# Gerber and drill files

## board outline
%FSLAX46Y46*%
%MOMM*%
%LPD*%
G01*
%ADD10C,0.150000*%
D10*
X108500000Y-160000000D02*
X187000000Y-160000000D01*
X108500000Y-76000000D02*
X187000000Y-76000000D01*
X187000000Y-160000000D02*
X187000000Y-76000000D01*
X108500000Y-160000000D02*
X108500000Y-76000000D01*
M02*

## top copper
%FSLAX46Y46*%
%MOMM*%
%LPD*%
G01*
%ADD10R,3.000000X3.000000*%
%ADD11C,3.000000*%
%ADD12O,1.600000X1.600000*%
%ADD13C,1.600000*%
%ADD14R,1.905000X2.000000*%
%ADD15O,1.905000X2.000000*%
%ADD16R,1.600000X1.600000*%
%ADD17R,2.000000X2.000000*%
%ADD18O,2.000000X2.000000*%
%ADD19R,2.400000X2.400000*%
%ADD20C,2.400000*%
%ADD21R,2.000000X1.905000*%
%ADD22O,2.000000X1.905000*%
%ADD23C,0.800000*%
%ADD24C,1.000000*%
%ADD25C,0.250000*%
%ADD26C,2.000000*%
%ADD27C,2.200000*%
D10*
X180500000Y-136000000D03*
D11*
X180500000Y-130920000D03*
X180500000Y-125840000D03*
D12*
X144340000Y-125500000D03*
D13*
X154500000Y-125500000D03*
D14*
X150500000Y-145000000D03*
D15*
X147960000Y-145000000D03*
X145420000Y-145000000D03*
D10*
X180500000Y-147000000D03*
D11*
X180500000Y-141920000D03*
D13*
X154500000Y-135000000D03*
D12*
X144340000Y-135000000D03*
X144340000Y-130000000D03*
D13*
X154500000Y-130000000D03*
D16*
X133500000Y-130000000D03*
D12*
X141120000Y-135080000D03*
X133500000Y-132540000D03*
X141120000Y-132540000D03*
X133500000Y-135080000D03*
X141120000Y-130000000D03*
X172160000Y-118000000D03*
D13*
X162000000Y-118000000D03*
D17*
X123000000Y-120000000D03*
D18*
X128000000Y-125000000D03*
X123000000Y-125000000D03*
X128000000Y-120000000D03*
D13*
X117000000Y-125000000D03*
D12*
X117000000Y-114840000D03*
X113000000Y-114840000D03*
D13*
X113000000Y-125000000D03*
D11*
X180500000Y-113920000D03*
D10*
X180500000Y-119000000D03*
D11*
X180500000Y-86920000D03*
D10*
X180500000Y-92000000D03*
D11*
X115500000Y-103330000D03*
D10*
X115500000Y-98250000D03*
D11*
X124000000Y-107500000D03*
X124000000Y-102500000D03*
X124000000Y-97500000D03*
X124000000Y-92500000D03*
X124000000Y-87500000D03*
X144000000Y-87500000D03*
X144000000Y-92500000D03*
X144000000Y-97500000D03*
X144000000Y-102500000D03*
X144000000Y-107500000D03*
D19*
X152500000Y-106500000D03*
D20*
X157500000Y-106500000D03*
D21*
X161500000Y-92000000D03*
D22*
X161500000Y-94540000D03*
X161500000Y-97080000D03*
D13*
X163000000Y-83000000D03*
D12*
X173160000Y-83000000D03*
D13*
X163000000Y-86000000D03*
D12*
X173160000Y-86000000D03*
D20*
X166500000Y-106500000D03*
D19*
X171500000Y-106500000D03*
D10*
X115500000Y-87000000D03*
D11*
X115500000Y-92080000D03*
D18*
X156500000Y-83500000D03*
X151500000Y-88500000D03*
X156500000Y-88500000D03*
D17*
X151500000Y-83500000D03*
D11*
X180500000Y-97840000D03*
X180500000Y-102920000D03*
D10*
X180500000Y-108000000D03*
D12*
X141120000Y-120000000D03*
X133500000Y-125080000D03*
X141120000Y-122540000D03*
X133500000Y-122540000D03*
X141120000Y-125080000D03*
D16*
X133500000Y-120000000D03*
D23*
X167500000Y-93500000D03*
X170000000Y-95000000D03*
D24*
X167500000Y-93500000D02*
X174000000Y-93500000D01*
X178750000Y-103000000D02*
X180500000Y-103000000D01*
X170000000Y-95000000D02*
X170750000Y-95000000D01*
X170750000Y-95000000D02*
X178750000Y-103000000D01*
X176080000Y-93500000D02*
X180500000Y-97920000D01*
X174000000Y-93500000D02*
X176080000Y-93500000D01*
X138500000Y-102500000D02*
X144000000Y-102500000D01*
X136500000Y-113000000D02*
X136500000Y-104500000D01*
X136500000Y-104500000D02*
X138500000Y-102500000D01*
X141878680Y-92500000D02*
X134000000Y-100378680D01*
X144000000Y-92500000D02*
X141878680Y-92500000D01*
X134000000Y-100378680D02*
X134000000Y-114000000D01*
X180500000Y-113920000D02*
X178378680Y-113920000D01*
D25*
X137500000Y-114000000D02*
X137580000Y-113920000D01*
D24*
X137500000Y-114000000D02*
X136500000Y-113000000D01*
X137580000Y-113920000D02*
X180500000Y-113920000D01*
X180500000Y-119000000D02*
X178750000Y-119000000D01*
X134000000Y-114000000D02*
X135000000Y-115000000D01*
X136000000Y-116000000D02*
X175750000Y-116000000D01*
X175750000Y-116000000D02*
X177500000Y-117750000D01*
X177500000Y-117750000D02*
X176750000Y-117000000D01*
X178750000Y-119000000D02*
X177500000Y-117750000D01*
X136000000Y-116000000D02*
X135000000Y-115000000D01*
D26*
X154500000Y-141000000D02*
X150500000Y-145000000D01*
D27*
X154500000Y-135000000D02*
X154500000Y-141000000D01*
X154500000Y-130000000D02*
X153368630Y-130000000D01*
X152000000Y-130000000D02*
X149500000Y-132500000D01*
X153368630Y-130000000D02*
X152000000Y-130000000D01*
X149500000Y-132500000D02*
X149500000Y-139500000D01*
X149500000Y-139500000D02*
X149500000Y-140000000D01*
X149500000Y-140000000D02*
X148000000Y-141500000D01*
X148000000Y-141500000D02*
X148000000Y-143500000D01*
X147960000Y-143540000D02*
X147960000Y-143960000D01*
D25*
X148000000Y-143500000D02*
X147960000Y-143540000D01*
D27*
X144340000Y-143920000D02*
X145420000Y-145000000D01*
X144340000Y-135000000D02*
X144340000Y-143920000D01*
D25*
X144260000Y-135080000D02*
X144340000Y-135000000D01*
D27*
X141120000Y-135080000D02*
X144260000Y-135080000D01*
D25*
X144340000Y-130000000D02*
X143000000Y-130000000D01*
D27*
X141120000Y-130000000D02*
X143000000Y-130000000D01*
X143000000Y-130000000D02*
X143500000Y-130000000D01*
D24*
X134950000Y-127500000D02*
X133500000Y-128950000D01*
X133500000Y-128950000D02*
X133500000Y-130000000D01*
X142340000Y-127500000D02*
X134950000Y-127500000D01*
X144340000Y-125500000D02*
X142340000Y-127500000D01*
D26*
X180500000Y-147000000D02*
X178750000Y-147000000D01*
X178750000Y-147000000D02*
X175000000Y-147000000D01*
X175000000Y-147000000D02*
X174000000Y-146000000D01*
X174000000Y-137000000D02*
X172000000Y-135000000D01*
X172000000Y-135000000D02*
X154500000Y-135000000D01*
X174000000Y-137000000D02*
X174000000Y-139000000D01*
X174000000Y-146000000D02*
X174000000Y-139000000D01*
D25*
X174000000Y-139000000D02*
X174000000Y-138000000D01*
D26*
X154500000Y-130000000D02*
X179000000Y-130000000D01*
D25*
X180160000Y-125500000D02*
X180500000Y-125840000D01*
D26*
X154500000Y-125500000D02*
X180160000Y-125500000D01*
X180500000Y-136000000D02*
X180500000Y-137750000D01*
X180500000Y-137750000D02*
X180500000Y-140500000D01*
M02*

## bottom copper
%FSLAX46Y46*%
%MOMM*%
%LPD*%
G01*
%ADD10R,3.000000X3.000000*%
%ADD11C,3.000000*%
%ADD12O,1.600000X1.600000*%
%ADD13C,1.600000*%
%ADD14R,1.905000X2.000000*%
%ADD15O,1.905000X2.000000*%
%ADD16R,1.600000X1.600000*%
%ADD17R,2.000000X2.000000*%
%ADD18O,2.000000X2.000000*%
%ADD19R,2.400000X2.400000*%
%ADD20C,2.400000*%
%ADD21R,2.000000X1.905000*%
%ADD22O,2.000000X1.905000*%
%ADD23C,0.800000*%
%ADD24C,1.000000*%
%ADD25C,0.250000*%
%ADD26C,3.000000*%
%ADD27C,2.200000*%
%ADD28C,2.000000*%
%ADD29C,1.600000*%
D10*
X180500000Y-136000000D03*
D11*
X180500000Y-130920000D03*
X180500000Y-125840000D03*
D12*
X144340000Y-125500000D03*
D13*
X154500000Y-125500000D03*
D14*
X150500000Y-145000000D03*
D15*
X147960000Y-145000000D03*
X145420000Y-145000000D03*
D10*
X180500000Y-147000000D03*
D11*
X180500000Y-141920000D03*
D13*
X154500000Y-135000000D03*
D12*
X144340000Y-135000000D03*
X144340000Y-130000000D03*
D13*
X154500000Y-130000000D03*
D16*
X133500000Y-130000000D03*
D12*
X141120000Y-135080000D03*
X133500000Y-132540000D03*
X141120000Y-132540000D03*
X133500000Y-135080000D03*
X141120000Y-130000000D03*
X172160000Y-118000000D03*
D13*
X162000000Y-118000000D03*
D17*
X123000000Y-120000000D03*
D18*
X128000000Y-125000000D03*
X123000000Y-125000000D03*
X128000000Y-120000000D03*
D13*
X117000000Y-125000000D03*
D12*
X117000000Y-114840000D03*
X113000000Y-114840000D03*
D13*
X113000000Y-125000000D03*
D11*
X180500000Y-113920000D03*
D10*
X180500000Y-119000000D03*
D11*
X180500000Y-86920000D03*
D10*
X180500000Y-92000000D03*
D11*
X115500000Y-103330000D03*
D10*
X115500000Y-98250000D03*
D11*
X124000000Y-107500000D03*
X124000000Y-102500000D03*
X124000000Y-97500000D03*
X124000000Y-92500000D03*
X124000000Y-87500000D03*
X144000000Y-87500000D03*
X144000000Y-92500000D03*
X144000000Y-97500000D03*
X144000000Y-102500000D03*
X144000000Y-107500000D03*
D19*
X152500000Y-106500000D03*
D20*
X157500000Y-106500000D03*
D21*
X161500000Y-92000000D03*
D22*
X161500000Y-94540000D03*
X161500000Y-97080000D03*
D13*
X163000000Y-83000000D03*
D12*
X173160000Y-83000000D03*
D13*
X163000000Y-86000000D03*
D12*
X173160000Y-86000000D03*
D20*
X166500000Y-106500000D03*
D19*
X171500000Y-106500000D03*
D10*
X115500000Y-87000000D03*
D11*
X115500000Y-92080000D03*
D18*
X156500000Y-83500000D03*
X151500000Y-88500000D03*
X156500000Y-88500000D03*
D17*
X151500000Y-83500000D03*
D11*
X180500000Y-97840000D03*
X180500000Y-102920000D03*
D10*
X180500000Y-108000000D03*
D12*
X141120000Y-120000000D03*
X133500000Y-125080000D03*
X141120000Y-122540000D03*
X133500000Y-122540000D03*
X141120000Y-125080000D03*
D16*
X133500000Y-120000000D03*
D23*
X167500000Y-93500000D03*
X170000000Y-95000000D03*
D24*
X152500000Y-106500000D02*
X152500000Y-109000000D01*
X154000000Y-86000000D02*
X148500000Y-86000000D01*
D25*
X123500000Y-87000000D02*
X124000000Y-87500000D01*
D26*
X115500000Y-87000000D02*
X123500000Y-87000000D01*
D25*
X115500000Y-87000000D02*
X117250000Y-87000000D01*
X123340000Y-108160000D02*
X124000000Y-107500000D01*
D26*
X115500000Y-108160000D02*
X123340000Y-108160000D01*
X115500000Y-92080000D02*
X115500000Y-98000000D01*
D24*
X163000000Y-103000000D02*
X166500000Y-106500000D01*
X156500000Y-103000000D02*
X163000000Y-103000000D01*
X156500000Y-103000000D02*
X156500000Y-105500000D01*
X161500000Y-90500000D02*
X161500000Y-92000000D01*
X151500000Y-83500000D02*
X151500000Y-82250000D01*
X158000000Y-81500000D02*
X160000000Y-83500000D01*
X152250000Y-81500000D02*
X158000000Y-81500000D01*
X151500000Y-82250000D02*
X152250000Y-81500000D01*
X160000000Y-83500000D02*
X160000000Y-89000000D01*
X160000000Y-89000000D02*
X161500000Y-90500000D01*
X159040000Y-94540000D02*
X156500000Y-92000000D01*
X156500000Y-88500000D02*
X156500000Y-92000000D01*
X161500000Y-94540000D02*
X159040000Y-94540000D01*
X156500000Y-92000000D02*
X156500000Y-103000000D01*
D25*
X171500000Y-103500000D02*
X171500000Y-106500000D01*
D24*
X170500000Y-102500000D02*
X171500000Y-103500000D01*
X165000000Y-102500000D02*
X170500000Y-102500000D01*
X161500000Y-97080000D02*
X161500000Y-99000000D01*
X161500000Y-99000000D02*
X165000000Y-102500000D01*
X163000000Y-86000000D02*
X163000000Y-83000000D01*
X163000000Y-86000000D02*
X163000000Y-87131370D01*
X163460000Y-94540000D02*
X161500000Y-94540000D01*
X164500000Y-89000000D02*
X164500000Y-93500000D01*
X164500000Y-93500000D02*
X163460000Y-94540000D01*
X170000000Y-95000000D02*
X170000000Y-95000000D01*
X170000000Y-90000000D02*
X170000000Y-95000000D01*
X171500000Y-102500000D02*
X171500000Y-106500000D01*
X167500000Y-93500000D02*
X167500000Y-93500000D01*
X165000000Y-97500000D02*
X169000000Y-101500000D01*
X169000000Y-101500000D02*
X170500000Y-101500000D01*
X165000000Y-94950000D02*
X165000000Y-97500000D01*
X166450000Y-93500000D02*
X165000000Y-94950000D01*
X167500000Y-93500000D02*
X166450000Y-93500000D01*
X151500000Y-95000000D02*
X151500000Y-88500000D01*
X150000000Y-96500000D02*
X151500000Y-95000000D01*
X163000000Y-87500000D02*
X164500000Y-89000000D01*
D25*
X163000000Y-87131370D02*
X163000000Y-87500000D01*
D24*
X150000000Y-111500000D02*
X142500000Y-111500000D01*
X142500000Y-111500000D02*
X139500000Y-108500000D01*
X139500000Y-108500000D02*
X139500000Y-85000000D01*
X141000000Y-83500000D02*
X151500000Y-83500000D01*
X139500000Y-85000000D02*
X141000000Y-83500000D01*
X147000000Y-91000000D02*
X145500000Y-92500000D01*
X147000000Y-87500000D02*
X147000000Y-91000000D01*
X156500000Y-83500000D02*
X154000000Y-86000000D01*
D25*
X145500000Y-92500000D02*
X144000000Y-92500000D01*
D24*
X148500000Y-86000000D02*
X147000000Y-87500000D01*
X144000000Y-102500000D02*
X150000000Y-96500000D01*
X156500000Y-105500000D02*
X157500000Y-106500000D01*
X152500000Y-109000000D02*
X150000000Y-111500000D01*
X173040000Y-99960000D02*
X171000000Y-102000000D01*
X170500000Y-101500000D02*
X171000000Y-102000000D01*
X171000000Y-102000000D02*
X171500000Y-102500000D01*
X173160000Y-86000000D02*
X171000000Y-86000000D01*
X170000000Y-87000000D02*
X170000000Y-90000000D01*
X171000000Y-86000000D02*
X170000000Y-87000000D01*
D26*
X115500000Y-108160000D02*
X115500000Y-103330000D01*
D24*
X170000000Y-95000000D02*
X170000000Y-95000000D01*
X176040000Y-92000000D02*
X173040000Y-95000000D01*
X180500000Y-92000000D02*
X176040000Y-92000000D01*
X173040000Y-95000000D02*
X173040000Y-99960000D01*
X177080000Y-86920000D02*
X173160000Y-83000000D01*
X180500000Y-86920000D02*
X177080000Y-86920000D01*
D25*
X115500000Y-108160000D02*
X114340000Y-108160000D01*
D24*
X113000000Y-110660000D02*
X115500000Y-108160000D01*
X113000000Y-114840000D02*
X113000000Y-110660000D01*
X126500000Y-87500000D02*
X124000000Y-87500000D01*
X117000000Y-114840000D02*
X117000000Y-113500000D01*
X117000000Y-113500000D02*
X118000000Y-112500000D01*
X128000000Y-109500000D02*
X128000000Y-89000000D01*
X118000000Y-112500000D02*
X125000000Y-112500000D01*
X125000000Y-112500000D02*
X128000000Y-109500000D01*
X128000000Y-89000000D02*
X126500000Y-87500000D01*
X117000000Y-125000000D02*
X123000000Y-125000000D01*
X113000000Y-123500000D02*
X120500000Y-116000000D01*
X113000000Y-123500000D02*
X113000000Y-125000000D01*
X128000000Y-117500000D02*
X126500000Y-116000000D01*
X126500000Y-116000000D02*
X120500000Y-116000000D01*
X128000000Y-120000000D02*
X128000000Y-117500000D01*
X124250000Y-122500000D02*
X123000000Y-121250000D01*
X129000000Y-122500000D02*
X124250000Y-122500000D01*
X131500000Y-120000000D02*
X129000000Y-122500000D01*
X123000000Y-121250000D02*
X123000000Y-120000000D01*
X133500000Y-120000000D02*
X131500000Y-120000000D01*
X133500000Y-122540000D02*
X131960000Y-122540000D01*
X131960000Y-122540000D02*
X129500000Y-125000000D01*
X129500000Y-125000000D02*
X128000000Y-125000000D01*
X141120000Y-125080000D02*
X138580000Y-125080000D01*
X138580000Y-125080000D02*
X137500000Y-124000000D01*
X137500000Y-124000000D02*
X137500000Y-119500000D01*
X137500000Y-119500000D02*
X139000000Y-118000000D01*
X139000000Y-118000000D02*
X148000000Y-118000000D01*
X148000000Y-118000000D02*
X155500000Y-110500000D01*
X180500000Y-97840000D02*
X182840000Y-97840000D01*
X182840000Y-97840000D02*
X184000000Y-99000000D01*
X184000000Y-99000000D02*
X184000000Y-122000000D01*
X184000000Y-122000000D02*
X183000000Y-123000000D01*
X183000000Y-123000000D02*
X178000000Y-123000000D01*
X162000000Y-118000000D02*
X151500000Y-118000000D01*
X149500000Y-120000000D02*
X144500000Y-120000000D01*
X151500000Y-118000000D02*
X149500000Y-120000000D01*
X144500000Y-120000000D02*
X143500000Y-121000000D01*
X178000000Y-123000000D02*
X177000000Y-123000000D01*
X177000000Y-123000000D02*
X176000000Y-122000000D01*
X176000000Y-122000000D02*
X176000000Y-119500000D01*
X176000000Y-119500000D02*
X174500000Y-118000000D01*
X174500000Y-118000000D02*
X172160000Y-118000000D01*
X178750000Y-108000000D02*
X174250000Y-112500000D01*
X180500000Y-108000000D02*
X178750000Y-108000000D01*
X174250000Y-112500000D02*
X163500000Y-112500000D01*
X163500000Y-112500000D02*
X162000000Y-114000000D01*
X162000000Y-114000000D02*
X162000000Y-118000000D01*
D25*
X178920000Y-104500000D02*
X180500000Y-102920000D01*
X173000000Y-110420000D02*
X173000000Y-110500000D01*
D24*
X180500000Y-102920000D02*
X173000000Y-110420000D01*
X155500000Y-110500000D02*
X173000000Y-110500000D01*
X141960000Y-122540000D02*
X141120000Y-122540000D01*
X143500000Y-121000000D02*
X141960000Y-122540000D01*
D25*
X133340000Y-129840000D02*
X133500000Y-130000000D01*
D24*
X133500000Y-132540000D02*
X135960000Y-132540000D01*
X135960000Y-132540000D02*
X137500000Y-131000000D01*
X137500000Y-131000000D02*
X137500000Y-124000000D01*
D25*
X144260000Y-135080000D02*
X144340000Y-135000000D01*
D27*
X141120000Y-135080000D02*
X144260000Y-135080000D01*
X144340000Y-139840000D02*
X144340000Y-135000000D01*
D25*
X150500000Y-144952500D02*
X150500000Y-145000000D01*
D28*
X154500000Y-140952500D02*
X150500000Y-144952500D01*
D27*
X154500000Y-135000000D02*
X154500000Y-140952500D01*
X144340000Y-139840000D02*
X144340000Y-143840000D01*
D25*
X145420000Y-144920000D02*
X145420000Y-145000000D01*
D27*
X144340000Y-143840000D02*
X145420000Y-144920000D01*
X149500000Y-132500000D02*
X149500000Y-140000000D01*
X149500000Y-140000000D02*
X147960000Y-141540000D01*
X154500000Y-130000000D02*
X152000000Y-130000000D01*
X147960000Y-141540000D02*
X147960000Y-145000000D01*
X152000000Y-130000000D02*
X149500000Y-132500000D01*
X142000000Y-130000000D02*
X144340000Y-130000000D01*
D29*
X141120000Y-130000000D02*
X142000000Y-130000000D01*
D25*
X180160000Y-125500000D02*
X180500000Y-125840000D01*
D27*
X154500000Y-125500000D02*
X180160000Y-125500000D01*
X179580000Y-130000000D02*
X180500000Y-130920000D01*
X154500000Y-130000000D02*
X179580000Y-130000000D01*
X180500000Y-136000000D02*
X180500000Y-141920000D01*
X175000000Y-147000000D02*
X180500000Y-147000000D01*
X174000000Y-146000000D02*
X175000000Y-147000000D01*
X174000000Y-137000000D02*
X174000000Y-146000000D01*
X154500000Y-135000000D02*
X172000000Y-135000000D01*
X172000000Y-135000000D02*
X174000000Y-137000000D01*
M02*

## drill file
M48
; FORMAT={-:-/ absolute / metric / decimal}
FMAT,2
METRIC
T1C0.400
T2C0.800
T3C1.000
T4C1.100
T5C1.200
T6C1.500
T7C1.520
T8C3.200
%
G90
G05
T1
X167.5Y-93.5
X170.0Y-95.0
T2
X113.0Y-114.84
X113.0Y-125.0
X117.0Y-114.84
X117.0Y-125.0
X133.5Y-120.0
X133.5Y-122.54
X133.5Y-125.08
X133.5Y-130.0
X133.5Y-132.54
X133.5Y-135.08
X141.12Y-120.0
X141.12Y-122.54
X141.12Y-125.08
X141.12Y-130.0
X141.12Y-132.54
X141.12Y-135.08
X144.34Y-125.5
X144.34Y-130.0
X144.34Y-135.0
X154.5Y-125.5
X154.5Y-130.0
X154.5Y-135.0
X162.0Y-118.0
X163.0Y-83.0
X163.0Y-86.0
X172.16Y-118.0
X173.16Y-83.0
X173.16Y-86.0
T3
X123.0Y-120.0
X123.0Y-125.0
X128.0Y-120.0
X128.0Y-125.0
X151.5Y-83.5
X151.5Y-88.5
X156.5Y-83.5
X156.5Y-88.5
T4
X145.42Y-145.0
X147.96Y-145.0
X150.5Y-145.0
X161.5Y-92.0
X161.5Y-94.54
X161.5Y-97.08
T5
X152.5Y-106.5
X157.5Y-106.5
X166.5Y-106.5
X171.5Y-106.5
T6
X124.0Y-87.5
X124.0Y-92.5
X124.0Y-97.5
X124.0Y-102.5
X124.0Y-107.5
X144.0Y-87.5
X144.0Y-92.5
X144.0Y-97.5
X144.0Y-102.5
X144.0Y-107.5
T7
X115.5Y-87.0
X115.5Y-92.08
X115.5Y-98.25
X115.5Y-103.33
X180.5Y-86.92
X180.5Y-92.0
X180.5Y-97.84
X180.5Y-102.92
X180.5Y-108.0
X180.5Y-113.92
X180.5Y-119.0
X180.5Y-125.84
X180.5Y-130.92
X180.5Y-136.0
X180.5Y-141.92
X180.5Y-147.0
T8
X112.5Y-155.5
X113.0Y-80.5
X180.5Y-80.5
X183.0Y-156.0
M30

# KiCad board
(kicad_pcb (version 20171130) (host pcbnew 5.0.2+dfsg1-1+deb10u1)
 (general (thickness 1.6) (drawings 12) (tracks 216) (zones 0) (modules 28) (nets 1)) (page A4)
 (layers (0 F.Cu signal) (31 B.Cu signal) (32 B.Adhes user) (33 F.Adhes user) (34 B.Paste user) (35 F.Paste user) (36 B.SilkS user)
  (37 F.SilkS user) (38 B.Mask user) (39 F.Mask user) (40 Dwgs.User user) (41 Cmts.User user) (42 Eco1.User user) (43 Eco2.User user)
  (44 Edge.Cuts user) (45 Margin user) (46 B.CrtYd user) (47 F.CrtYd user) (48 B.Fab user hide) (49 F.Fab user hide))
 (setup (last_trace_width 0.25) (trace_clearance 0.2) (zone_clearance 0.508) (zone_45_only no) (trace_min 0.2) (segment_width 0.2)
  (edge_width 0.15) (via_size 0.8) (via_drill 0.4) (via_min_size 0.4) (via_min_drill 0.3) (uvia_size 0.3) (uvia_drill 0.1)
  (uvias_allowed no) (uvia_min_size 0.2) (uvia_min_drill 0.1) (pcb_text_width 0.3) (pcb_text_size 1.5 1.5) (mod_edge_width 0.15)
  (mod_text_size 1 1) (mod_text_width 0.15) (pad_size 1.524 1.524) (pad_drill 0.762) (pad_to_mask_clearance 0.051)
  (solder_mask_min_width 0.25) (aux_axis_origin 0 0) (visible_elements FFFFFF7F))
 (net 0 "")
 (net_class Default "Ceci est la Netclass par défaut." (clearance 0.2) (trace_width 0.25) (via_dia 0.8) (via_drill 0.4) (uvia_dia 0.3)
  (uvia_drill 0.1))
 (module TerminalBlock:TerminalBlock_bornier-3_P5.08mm (layer F.Cu) (at 180.5 136 90)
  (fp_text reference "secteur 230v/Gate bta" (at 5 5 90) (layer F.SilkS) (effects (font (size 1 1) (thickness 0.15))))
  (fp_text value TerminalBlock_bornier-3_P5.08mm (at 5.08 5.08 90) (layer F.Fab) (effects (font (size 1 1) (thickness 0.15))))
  (pad 1 thru_hole rect (at 0 0 90) (size 3 3) (drill 1.52) (layers *.Cu *.Mask))
  (pad 2 thru_hole circle (at 5.08 0 90) (size 3 3) (drill 1.52) (layers *.Cu *.Mask))
  (pad 3 thru_hole circle (at 10.16 0 90) (size 3 3) (drill 1.52) (layers *.Cu *.Mask)))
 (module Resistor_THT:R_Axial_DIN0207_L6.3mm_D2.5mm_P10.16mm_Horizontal (layer F.Cu) (at 154.5 125.5 180)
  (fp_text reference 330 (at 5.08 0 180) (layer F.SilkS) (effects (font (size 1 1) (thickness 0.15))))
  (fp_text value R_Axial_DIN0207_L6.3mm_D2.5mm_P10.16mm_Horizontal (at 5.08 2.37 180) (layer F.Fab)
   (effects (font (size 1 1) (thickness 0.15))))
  (pad 2 thru_hole oval (at 10.16 0 180) (size 1.6 1.6) (drill 0.8) (layers *.Cu *.Mask))
  (pad 1 thru_hole circle (at 0 0 180) (size 1.6 1.6) (drill 0.8) (layers *.Cu *.Mask)))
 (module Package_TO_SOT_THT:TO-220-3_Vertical (layer F.Cu) (at 150.5 145 180)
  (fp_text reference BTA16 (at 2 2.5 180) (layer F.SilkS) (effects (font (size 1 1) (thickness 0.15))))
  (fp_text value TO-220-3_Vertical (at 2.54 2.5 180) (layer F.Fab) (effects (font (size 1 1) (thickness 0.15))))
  (pad 1 thru_hole rect (at 0 0 180) (size 1.905 2) (drill 1.1) (layers *.Cu *.Mask))
  (pad 2 thru_hole oval (at 2.54 0 180) (size 1.905 2) (drill 1.1) (layers *.Cu *.Mask))
  (pad 3 thru_hole oval (at 5.08 0 180) (size 1.905 2) (drill 1.1) (layers *.Cu *.Mask)))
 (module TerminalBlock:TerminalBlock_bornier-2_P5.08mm (layer F.Cu) (at 180.5 147 90)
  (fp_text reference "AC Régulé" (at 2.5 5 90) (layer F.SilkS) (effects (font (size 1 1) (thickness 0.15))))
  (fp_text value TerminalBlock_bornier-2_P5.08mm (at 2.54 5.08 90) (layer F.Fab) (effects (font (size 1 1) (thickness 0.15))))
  (pad 1 thru_hole rect (at 0 0 90) (size 3 3) (drill 1.52) (layers *.Cu *.Mask))
  (pad 2 thru_hole circle (at 5.08 0 90) (size 3 3) (drill 1.52) (layers *.Cu *.Mask)))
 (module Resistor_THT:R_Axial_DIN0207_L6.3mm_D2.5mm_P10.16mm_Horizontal (layer F.Cu) (at 154.5 135 180)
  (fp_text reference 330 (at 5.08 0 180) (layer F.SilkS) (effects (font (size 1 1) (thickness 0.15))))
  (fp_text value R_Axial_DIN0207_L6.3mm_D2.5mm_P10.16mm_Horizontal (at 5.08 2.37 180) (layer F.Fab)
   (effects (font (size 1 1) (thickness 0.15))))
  (pad 1 thru_hole circle (at 0 0 180) (size 1.6 1.6) (drill 0.8) (layers *.Cu *.Mask))
  (pad 2 thru_hole oval (at 10.16 0 180) (size 1.6 1.6) (drill 0.8) (layers *.Cu *.Mask)))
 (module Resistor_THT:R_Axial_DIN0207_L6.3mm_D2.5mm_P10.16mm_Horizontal (layer F.Cu) (at 154.5 130 180)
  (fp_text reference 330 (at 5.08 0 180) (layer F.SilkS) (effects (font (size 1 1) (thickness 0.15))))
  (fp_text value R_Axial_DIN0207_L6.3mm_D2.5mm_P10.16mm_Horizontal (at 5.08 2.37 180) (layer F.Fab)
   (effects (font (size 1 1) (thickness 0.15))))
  (pad 2 thru_hole oval (at 10.16 0 180) (size 1.6 1.6) (drill 0.8) (layers *.Cu *.Mask))
  (pad 1 thru_hole circle (at 0 0 180) (size 1.6 1.6) (drill 0.8) (layers *.Cu *.Mask)))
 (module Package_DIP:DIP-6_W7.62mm (layer F.Cu) (at 133.5 130)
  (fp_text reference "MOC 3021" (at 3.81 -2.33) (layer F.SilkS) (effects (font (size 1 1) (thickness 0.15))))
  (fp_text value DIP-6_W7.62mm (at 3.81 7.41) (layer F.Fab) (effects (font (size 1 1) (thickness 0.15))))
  (pad 1 thru_hole rect (at 0 0) (size 1.6 1.6) (drill 0.8) (layers *.Cu *.Mask))
  (pad 4 thru_hole oval (at 7.62 5.08) (size 1.6 1.6) (drill 0.8) (layers *.Cu *.Mask))
  (pad 2 thru_hole oval (at 0 2.54) (size 1.6 1.6) (drill 0.8) (layers *.Cu *.Mask))
  (pad 5 thru_hole oval (at 7.62 2.54) (size 1.6 1.6) (drill 0.8) (layers *.Cu *.Mask))
  (pad 3 thru_hole oval (at 0 5.08) (size 1.6 1.6) (drill 0.8) (layers *.Cu *.Mask))
  (pad 6 thru_hole oval (at 7.62 0) (size 1.6 1.6) (drill 0.8) (layers *.Cu *.Mask)))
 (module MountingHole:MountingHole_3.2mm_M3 (layer F.Cu) (at 183 156)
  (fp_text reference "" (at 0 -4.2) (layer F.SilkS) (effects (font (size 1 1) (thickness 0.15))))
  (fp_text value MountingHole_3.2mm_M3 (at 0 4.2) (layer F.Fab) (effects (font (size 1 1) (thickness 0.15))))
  (pad 1 np_thru_hole circle (at 0 0) (size 3.2 3.2) (drill 3.2) (layers *.Cu *.Mask)))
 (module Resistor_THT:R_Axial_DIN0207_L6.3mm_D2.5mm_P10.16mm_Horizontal (layer F.Cu) (at 162 118)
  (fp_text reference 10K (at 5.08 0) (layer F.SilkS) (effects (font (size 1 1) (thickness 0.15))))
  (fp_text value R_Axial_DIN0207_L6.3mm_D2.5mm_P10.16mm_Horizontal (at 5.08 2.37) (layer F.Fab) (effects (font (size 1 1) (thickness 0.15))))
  (pad 2 thru_hole oval (at 10.16 0) (size 1.6 1.6) (drill 0.8) (layers *.Cu *.Mask))
  (pad 1 thru_hole circle (at 0 0) (size 1.6 1.6) (drill 0.8) (layers *.Cu *.Mask)))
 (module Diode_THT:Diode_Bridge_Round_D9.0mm (layer F.Cu) (at 123 120)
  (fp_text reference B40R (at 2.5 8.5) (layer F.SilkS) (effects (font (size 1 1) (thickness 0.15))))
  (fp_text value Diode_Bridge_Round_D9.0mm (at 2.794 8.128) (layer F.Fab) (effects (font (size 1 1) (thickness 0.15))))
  (pad 1 thru_hole rect (at 0 0) (size 2 2) (drill 1) (layers *.Cu *.Mask))
  (pad 3 thru_hole oval (at 5 5) (size 2 2) (drill 1) (layers *.Cu *.Mask))
  (pad 2 thru_hole oval (at 0 5) (size 2 2) (drill 1) (layers *.Cu *.Mask))
  (pad 4 thru_hole oval (at 5 0) (size 2 2) (drill 1) (layers *.Cu *.Mask)))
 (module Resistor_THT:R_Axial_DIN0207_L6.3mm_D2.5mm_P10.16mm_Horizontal (layer F.Cu) (at 117 125 90)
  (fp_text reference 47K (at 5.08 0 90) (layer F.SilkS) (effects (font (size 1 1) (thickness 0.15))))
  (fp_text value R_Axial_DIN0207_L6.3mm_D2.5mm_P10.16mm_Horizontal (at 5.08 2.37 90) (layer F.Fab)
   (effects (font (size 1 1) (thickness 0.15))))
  (pad 1 thru_hole circle (at 0 0 90) (size 1.6 1.6) (drill 0.8) (layers *.Cu *.Mask))
  (pad 2 thru_hole oval (at 10.16 0 90) (size 1.6 1.6) (drill 0.8) (layers *.Cu *.Mask)))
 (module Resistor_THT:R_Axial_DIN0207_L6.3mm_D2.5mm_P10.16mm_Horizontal (layer F.Cu) (at 113 125 90)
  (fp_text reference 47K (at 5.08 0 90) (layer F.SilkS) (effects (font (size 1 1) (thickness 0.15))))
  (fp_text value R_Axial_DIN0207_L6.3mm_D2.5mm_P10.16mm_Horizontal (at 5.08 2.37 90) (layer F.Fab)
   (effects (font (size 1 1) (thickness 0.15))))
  (pad 2 thru_hole oval (at 10.16 0 90) (size 1.6 1.6) (drill 0.8) (layers *.Cu *.Mask))
  (pad 1 thru_hole circle (at 0 0 90) (size 1.6 1.6) (drill 0.8) (layers *.Cu *.Mask)))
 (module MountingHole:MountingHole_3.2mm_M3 (layer F.Cu) (at 180.5 80.5)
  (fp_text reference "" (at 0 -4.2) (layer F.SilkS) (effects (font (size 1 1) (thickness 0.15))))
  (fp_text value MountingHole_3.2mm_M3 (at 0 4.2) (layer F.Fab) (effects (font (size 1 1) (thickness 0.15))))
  (pad 1 np_thru_hole circle (at 0 0) (size 3.2 3.2) (drill 3.2) (layers *.Cu *.Mask)))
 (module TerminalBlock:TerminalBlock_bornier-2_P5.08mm (layer F.Cu) (at 180.5 119 90)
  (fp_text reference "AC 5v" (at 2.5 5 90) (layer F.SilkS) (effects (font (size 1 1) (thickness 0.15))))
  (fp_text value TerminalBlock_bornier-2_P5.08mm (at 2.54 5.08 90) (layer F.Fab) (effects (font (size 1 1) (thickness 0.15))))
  (pad 2 thru_hole circle (at 5.08 0 90) (size 3 3) (drill 1.52) (layers *.Cu *.Mask))
  (pad 1 thru_hole rect (at 0 0 90) (size 3 3) (drill 1.52) (layers *.Cu *.Mask)))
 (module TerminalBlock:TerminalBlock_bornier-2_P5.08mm (layer F.Cu) (at 180.5 92 90)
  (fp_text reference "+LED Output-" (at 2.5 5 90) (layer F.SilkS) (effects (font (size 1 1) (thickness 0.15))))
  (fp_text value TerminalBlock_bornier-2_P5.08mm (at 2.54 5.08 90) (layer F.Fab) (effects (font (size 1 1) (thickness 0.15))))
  (pad 2 thru_hole circle (at 5.08 0 90) (size 3 3) (drill 1.52) (layers *.Cu *.Mask))
  (pad 1 thru_hole rect (at 0 0 90) (size 3 3) (drill 1.52) (layers *.Cu *.Mask)))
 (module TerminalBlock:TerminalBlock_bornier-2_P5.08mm (layer F.Cu) (at 115.5 98.25 270)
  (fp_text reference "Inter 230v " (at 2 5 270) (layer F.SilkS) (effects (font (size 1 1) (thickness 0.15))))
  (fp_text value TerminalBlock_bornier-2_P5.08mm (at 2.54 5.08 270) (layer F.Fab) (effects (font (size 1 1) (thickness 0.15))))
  (pad 2 thru_hole circle (at 5.08 0 270) (size 3 3) (drill 1.52) (layers *.Cu *.Mask))
  (pad 1 thru_hole rect (at 0 0 270) (size 3 3) (drill 1.52) (layers *.Cu *.Mask)))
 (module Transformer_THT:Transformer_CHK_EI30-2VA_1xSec (layer F.Cu) (at 124 107.5)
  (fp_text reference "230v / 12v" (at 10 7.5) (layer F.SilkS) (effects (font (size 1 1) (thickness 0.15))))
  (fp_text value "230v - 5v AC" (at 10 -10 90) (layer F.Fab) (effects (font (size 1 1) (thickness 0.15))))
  (pad 1 thru_hole circle (at 0 0) (size 3 3) (drill 1.5) (layers *.Cu *.Mask))
  (pad 2 thru_hole circle (at 0 -5) (size 3 3) (drill 1.5) (layers *.Cu *.Mask))
  (pad 3 thru_hole circle (at 0 -10) (size 3 3) (drill 1.5) (layers *.Cu *.Mask))
  (pad 4 thru_hole circle (at 0 -15) (size 3 3) (drill 1.5) (layers *.Cu *.Mask))
  (pad 5 thru_hole circle (at 0 -20) (size 3 3) (drill 1.5) (layers *.Cu *.Mask))
  (pad 6 thru_hole circle (at 20 -20) (size 3 3) (drill 1.5) (layers *.Cu *.Mask))
  (pad 7 thru_hole circle (at 20 -15) (size 3 3) (drill 1.5) (layers *.Cu *.Mask))
  (pad 8 thru_hole circle (at 20 -10) (size 3 3) (drill 1.5) (layers *.Cu *.Mask))
  (pad 9 thru_hole circle (at 20 -5) (size 3 3) (drill 1.5) (layers *.Cu *.Mask))
  (pad 10 thru_hole circle (at 20 0) (size 3 3) (drill 1.5) (layers *.Cu *.Mask)))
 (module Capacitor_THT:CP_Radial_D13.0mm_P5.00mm (layer F.Cu) (at 152.5 106.5)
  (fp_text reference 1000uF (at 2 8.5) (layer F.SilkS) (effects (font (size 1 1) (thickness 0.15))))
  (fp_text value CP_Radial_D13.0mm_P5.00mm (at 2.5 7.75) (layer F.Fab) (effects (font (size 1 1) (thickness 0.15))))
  (pad 1 thru_hole rect (at 0 0) (size 2.4 2.4) (drill 1.2) (layers *.Cu *.Mask))
  (pad 2 thru_hole circle (at 5 0) (size 2.4 2.4) (drill 1.2) (layers *.Cu *.Mask)))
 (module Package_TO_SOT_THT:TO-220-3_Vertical (layer F.Cu) (at 161.5 92 270)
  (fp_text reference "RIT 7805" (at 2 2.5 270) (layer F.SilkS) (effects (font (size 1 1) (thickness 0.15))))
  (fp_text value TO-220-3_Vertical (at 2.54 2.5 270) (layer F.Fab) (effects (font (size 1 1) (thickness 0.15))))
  (pad 1 thru_hole rect (at 0 0 270) (size 1.905 2) (drill 1.1) (layers *.Cu *.Mask))
  (pad 2 thru_hole oval (at 2.54 0 270) (size 1.905 2) (drill 1.1) (layers *.Cu *.Mask))
  (pad 3 thru_hole oval (at 5.08 0 270) (size 1.905 2) (drill 1.1) (layers *.Cu *.Mask)))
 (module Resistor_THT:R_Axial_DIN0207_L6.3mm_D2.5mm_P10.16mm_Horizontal (layer F.Cu) (at 163 83)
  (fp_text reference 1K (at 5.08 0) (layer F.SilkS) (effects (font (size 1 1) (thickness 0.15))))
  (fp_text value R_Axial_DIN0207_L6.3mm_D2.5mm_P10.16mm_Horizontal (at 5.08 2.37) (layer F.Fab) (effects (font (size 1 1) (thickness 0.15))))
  (pad 1 thru_hole circle (at 0 0) (size 1.6 1.6) (drill 0.8) (layers *.Cu *.Mask))
  (pad 2 thru_hole oval (at 10.16 0) (size 1.6 1.6) (drill 0.8) (layers *.Cu *.Mask)))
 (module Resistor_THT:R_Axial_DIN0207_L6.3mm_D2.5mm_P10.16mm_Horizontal (layer F.Cu) (at 163 86)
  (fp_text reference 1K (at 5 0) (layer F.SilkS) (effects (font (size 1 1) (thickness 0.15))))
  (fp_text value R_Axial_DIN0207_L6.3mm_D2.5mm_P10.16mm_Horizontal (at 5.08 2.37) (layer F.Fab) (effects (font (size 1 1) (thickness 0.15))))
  (pad 1 thru_hole circle (at 0 0) (size 1.6 1.6) (drill 0.8) (layers *.Cu *.Mask))
  (pad 2 thru_hole oval (at 10.16 0) (size 1.6 1.6) (drill 0.8) (layers *.Cu *.Mask)))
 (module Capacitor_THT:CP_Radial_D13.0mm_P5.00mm (layer F.Cu) (at 171.5 106.5 180)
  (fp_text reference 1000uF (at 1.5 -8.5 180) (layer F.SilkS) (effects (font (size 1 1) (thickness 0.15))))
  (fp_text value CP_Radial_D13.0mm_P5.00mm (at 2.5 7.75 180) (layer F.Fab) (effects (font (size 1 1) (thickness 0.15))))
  (pad 2 thru_hole circle (at 5 0 180) (size 2.4 2.4) (drill 1.2) (layers *.Cu *.Mask))
  (pad 1 thru_hole rect (at 0 0 180) (size 2.4 2.4) (drill 1.2) (layers *.Cu *.Mask)))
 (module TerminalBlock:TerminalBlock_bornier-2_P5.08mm (layer F.Cu) (at 115.5 87 270)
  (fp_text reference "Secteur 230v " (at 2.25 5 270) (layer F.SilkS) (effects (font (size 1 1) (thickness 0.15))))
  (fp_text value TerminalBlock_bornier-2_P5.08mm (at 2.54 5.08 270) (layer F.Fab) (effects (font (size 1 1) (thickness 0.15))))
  (pad 1 thru_hole rect (at 0 0 270) (size 3 3) (drill 1.52) (layers *.Cu *.Mask))
  (pad 2 thru_hole circle (at 5.08 0 270) (size 3 3) (drill 1.52) (layers *.Cu *.Mask)))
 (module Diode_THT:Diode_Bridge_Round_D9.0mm (layer F.Cu) (at 151.5 83.5)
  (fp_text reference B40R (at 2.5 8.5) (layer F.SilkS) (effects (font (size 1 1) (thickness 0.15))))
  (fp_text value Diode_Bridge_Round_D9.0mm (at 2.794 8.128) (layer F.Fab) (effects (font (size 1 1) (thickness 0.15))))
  (pad 4 thru_hole oval (at 5 0) (size 2 2) (drill 1) (layers *.Cu *.Mask))
  (pad 2 thru_hole oval (at 0 5) (size 2 2) (drill 1) (layers *.Cu *.Mask))
  (pad 3 thru_hole oval (at 5 5) (size 2 2) (drill 1) (layers *.Cu *.Mask))
  (pad 1 thru_hole rect (at 0 0) (size 2 2) (drill 1) (layers *.Cu *.Mask)))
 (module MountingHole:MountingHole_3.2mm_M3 (layer F.Cu) (at 112.5 155.5)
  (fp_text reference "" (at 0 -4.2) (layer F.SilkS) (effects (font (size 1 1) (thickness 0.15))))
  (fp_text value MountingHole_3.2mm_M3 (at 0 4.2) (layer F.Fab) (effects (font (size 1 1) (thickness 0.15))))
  (pad 1 np_thru_hole circle (at 0 0) (size 3.2 3.2) (drill 3.2) (layers *.Cu *.Mask)))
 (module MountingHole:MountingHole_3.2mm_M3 (layer F.Cu) (at 113 80.5)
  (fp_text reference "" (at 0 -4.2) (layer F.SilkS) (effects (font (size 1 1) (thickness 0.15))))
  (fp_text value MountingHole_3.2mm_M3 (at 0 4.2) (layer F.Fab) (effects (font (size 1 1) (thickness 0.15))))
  (pad 1 np_thru_hole circle (at 0 0) (size 3.2 3.2) (drill 3.2) (layers *.Cu *.Mask)))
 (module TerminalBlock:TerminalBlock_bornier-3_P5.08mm (layer F.Cu) (at 180.5 108 90)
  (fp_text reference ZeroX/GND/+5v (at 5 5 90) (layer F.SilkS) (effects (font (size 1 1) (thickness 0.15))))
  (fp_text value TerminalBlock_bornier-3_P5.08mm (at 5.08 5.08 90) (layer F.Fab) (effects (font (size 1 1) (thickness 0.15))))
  (pad 3 thru_hole circle (at 10.16 0 90) (size 3 3) (drill 1.52) (layers *.Cu *.Mask))
  (pad 2 thru_hole circle (at 5.08 0 90) (size 3 3) (drill 1.52) (layers *.Cu *.Mask))
  (pad 1 thru_hole rect (at 0 0 90) (size 3 3) (drill 1.52) (layers *.Cu *.Mask)))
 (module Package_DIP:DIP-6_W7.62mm (layer F.Cu) (at 133.5 120)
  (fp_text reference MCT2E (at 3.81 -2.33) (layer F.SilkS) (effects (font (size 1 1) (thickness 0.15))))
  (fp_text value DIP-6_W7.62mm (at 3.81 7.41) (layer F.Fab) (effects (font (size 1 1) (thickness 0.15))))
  (pad 6 thru_hole oval (at 7.62 0) (size 1.6 1.6) (drill 0.8) (layers *.Cu *.Mask))
  (pad 3 thru_hole oval (at 0 5.08) (size 1.6 1.6) (drill 0.8) (layers *.Cu *.Mask))
  (pad 5 thru_hole oval (at 7.62 2.54) (size 1.6 1.6) (drill 0.8) (layers *.Cu *.Mask))
  (pad 2 thru_hole oval (at 0 2.54) (size 1.6 1.6) (drill 0.8) (layers *.Cu *.Mask))
  (pad 4 thru_hole oval (at 7.62 5.08) (size 1.6 1.6) (drill 0.8) (layers *.Cu *.Mask))
  (pad 1 thru_hole rect (at 0 0) (size 1.6 1.6) (drill 0.8) (layers *.Cu *.Mask)))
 (gr_line (start 108.5 160) (end 187 160) (layer Edge.Cuts) (width 0.15))
 (gr_line (start 108.5 76) (end 187 76) (layer Edge.Cuts) (width 0.15))
 (gr_line (start 187 160) (end 187 76) (layer Edge.Cuts) (width 0.15))
 (gr_line (start 108.5 160) (end 108.5 76) (layer Edge.Cuts) (width 0.15))
 (segment (start 152.5 106.5) (end 152.5 109) (width 1) (layer B.Cu) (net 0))
 (segment (start 154 86) (end 148.5 86) (width 1) (layer B.Cu) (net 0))
 (segment (start 123.5 87) (end 124 87.5) (width 0.25) (layer B.Cu) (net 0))
 (segment (start 115.5 87) (end 123.5 87) (width 3) (layer B.Cu) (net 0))
 (segment (start 115.5 87) (end 117.25 87) (width 0.25) (layer B.Cu) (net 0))
 (segment (start 123.34 108.16) (end 124 107.5) (width 0.25) (layer B.Cu) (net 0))
 (segment (start 115.5 108.16) (end 123.34 108.16) (width 3) (layer B.Cu) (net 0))
 (segment (start 115.5 92.08) (end 115.5 98) (width 3) (layer B.Cu) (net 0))
 (segment (start 163 103) (end 166.5 106.5) (width 1) (layer B.Cu) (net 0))
 (segment (start 156.5 103) (end 163 103) (width 1) (layer B.Cu) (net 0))
 (segment (start 156.5 103) (end 156.5 105.5) (width 1) (layer B.Cu) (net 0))
 (segment (start 161.5 90.5) (end 161.5 92) (width 1) (layer B.Cu) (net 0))
 (segment (start 151.5 83.5) (end 151.5 82.25) (width 1) (layer B.Cu) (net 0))
 (segment (start 158 81.5) (end 160 83.5) (width 1) (layer B.Cu) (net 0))
 (segment (start 152.25 81.5) (end 158 81.5) (width 1) (layer B.Cu) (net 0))
 (segment (start 151.5 82.25) (end 152.25 81.5) (width 1) (layer B.Cu) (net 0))
 (segment (start 160 83.5) (end 160 89) (width 1) (layer B.Cu) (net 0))
 (segment (start 160 89) (end 161.5 90.5) (width 1) (layer B.Cu) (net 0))
 (segment (start 159.04 94.54) (end 156.5 92) (width 1) (layer B.Cu) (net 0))
 (segment (start 156.5 88.5) (end 156.5 92) (width 1) (layer B.Cu) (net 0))
 (segment (start 161.5 94.54) (end 159.04 94.54) (width 1) (layer B.Cu) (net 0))
 (segment (start 156.5 92) (end 156.5 103) (width 1) (layer B.Cu) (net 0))
 (segment (start 171.5 103.5) (end 171.5 106.5) (width 0.25) (layer B.Cu) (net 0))
 (segment (start 170.5 102.5) (end 171.5 103.5) (width 1) (layer B.Cu) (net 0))
 (segment (start 165 102.5) (end 170.5 102.5) (width 1) (layer B.Cu) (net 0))
 (segment (start 161.5 97.08) (end 161.5 99) (width 1) (layer B.Cu) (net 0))
 (segment (start 161.5 99) (end 165 102.5) (width 1) (layer B.Cu) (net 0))
 (segment (start 163 86) (end 163 83) (width 1) (layer B.Cu) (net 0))
 (segment (start 163 86) (end 163 87.13137) (width 1) (layer B.Cu) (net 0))
 (segment (start 163.46 94.54) (end 161.5 94.54) (width 1) (layer B.Cu) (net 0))
 (segment (start 164.5 89) (end 164.5 93.5) (width 1) (layer B.Cu) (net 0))
 (segment (start 164.5 93.5) (end 163.46 94.54) (width 1) (layer B.Cu) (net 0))
 (segment (start 170 95) (end 170 95) (width 1) (layer B.Cu) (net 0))
 (segment (start 170 90) (end 170 95) (width 1) (layer B.Cu) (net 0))
 (segment (start 171.5 102.5) (end 171.5 106.5) (width 1) (layer B.Cu) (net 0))
 (segment (start 167.5 93.5) (end 167.5 93.5) (width 1) (layer B.Cu) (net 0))
 (segment (start 165 97.5) (end 169 101.5) (width 1) (layer B.Cu) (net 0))
 (segment (start 169 101.5) (end 170.5 101.5) (width 1) (layer B.Cu) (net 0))
 (segment (start 165 94.95) (end 165 97.5) (width 1) (layer B.Cu) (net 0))
 (segment (start 166.45 93.5) (end 165 94.95) (width 1) (layer B.Cu) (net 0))
 (segment (start 167.5 93.5) (end 166.45 93.5) (width 1) (layer B.Cu) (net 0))
 (via (at 167.5 93.5) (size 0.8) (drill 0.4) (layers F.Cu B.Cu) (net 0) (status 1000000))
 (segment (start 151.5 95) (end 151.5 88.5) (width 1) (layer B.Cu) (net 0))
 (segment (start 150 96.5) (end 151.5 95) (width 1) (layer B.Cu) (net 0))
 (segment (start 163 87.5) (end 164.5 89) (width 1) (layer B.Cu) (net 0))
 (segment (start 163 87.13137) (end 163 87.5) (width 0.25) (layer B.Cu) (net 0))
 (segment (start 150 111.5) (end 142.5 111.5) (width 1) (layer B.Cu) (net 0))
 (segment (start 142.5 111.5) (end 139.5 108.5) (width 1) (layer B.Cu) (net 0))
 (segment (start 139.5 108.5) (end 139.5 85) (width 1) (layer B.Cu) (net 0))
 (segment (start 141 83.5) (end 151.5 83.5) (width 1) (layer B.Cu) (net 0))
 (segment (start 139.5 85) (end 141 83.5) (width 1) (layer B.Cu) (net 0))
 (segment (start 147 91) (end 145.5 92.5) (width 1) (layer B.Cu) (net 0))
 (segment (start 147 87.5) (end 147 91) (width 1) (layer B.Cu) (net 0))
 (segment (start 156.5 83.5) (end 154 86) (width 1) (layer B.Cu) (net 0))
 (segment (start 145.5 92.5) (end 144 92.5) (width 0.25) (layer B.Cu) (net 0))
 (segment (start 148.5 86) (end 147 87.5) (width 1) (layer B.Cu) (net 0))
 (segment (start 144 102.5) (end 150 96.5) (width 1) (layer B.Cu) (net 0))
 (segment (start 156.5 105.5) (end 157.5 106.5) (width 1) (layer B.Cu) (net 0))
 (segment (start 152.5 109) (end 150 111.5) (width 1) (layer B.Cu) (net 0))
 (segment (start 173.04 99.96) (end 171 102) (width 1) (layer B.Cu) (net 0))
 (segment (start 170.5 101.5) (end 171 102) (width 1) (layer B.Cu) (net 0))
 (segment (start 171 102) (end 171.5 102.5) (width 1) (layer B.Cu) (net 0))
 (segment (start 173.16 86) (end 171 86) (width 1) (layer B.Cu) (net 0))
 (segment (start 170 87) (end 170 90) (width 1) (layer B.Cu) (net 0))
 (segment (start 171 86) (end 170 87) (width 1) (layer B.Cu) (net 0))
 (segment (start 115.5 108.16) (end 115.5 103.33) (width 3) (layer B.Cu) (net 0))
 (segment (start 167.5 93.5) (end 174 93.5) (width 1) (layer F.Cu) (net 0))
 (segment (start 170 95) (end 170 95) (width 1) (layer B.Cu) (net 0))
 (via (at 170 95) (size 0.8) (drill 0.4) (layers F.Cu B.Cu) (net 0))
 (segment (start 178.75 103) (end 180.5 103) (width 1) (layer F.Cu) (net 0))
 (segment (start 170 95) (end 170.75 95) (width 1) (layer F.Cu) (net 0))
 (segment (start 170.75 95) (end 178.75 103) (width 1) (layer F.Cu) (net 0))
 (segment (start 176.08 93.5) (end 180.5 97.92) (width 1) (layer F.Cu) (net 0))
 (segment (start 174 93.5) (end 176.08 93.5) (width 1) (layer F.Cu) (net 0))
 (segment (start 176.04 92) (end 173.04 95) (width 1) (layer B.Cu) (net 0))
 (segment (start 180.5 92) (end 176.04 92) (width 1) (layer B.Cu) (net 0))
 (segment (start 173.04 95) (end 173.04 99.96) (width 1) (layer B.Cu) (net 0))
 (segment (start 177.08 86.92) (end 173.16 83) (width 1) (layer B.Cu) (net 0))
 (segment (start 180.5 86.92) (end 177.08 86.92) (width 1) (layer B.Cu) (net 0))
 (segment (start 138.5 102.5) (end 144 102.5) (width 1) (layer F.Cu) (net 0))
 (segment (start 136.5 113) (end 136.5 104.5) (width 1) (layer F.Cu) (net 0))
 (segment (start 136.5 104.5) (end 138.5 102.5) (width 1) (layer F.Cu) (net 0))
 (segment (start 141.87868 92.5) (end 134 100.37868) (width 1) (layer F.Cu) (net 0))
 (segment (start 144 92.5) (end 141.87868 92.5) (width 1) (layer F.Cu) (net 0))
 (segment (start 134 100.37868) (end 134 114) (width 1) (layer F.Cu) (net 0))
 (segment (start 115.5 108.16) (end 114.34 108.16) (width 0.25) (layer B.Cu) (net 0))
 (segment (start 113 110.66) (end 115.5 108.16) (width 1) (layer B.Cu) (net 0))
 (segment (start 113 114.84) (end 113 110.66) (width 1) (layer B.Cu) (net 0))
 (segment (start 126.5 87.5) (end 124 87.5) (width 1) (layer B.Cu) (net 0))
 (segment (start 117 114.84) (end 117 113.5) (width 1) (layer B.Cu) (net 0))
 (segment (start 117 113.5) (end 118 112.5) (width 1) (layer B.Cu) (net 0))
 (segment (start 128 109.5) (end 128 89) (width 1) (layer B.Cu) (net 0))
 (segment (start 118 112.5) (end 125 112.5) (width 1) (layer B.Cu) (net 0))
 (segment (start 125 112.5) (end 128 109.5) (width 1) (layer B.Cu) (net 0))
 (segment (start 128 89) (end 126.5 87.5) (width 1) (layer B.Cu) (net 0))
 (segment (start 117 125) (end 123 125) (width 1) (layer B.Cu) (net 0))
 (segment (start 113 123.5) (end 120.5 116) (width 1) (layer B.Cu) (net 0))
 (segment (start 113 123.5) (end 113 125) (width 1) (layer B.Cu) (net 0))
 (segment (start 128 117.5) (end 126.5 116) (width 1) (layer B.Cu) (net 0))
 (segment (start 126.5 116) (end 120.5 116) (width 1) (layer B.Cu) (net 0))
 (segment (start 128 120) (end 128 117.5) (width 1) (layer B.Cu) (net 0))
 (segment (start 180.5 113.92) (end 178.37868 113.92) (width 1) (layer F.Cu) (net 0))
 (segment (start 137.5 114) (end 137.58 113.92) (width 0.25) (layer F.Cu) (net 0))
 (segment (start 137.5 114) (end 136.5 113) (width 1) (layer F.Cu) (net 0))
 (segment (start 137.58 113.92) (end 180.5 113.92) (width 1) (layer F.Cu) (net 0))
 (segment (start 180.5 119) (end 178.75 119) (width 1) (layer F.Cu) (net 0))
 (segment (start 134 114) (end 135 115) (width 1) (layer F.Cu) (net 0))
 (segment (start 136 116) (end 175.75 116) (width 1) (layer F.Cu) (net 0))
 (segment (start 175.75 116) (end 177.5 117.75) (width 1) (layer F.Cu) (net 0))
 (segment (start 177.5 117.75) (end 176.75 117) (width 1) (layer F.Cu) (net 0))
 (segment (start 178.75 119) (end 177.5 117.75) (width 1) (layer F.Cu) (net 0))
 (segment (start 136 116) (end 135 115) (width 1) (layer F.Cu) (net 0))
 (segment (start 124.25 122.5) (end 123 121.25) (width 1) (layer B.Cu) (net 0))
 (segment (start 129 122.5) (end 124.25 122.5) (width 1) (layer B.Cu) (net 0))
 (segment (start 131.5 120) (end 129 122.5) (width 1) (layer B.Cu) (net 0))
 (segment (start 123 121.25) (end 123 120) (width 1) (layer B.Cu) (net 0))
 (segment (start 133.5 120) (end 131.5 120) (width 1) (layer B.Cu) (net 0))
 (segment (start 133.5 122.54) (end 131.96 122.54) (width 1) (layer B.Cu) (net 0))
 (segment (start 131.96 122.54) (end 129.5 125) (width 1) (layer B.Cu) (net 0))
 (segment (start 129.5 125) (end 128 125) (width 1) (layer B.Cu) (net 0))
 (segment (start 141.12 125.08) (end 138.58 125.08) (width 1) (layer B.Cu) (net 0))
 (segment (start 138.58 125.08) (end 137.5 124) (width 1) (layer B.Cu) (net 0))
 (segment (start 137.5 124) (end 137.5 119.5) (width 1) (layer B.Cu) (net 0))
 (segment (start 137.5 119.5) (end 139 118) (width 1) (layer B.Cu) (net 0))
 (segment (start 139 118) (end 148 118) (width 1) (layer B.Cu) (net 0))
 (segment (start 148 118) (end 155.5 110.5) (width 1) (layer B.Cu) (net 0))
 (segment (start 180.5 97.84) (end 182.84 97.84) (width 1) (layer B.Cu) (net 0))
 (segment (start 182.84 97.84) (end 184 99) (width 1) (layer B.Cu) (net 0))
 (segment (start 184 99) (end 184 122) (width 1) (layer B.Cu) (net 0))
 (segment (start 184 122) (end 183 123) (width 1) (layer B.Cu) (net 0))
 (segment (start 183 123) (end 178 123) (width 1) (layer B.Cu) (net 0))
 (segment (start 162 118) (end 151.5 118) (width 1) (layer B.Cu) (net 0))
 (segment (start 149.5 120) (end 144.5 120) (width 1) (layer B.Cu) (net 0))
 (segment (start 151.5 118) (end 149.5 120) (width 1) (layer B.Cu) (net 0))
 (segment (start 144.5 120) (end 143.5 121) (width 1) (layer B.Cu) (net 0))
 (segment (start 178 123) (end 177 123) (width 1) (layer B.Cu) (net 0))
 (segment (start 177 123) (end 176 122) (width 1) (layer B.Cu) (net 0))
 (segment (start 176 122) (end 176 119.5) (width 1) (layer B.Cu) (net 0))
 (segment (start 176 119.5) (end 174.5 118) (width 1) (layer B.Cu) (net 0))
 (segment (start 174.5 118) (end 172.16 118) (width 1) (layer B.Cu) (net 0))
 (segment (start 178.75 108) (end 174.25 112.5) (width 1) (layer B.Cu) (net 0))
 (segment (start 180.5 108) (end 178.75 108) (width 1) (layer B.Cu) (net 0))
 (segment (start 174.25 112.5) (end 163.5 112.5) (width 1) (layer B.Cu) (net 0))
 (segment (start 163.5 112.5) (end 162 114) (width 1) (layer B.Cu) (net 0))
 (segment (start 162 114) (end 162 118) (width 1) (layer B.Cu) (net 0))
 (segment (start 178.92 104.5) (end 180.5 102.92) (width 0.25) (layer B.Cu) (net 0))
 (segment (start 173 110.42) (end 173 110.5) (width 0.25) (layer B.Cu) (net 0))
 (segment (start 180.5 102.92) (end 173 110.42) (width 1) (layer B.Cu) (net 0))
 (segment (start 155.5 110.5) (end 173 110.5) (width 1) (layer B.Cu) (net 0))
 (segment (start 141.96 122.54) (end 141.12 122.54) (width 1) (layer B.Cu) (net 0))
 (segment (start 143.5 121) (end 141.96 122.54) (width 1) (layer B.Cu) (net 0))
 (segment (start 133.34 129.84) (end 133.5 130) (width 0.25) (layer B.Cu) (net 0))
 (segment (start 133.5 132.54) (end 135.96 132.54) (width 1) (layer B.Cu) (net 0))
 (segment (start 135.96 132.54) (end 137.5 131) (width 1) (layer B.Cu) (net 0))
 (segment (start 137.5 131) (end 137.5 124) (width 1) (layer B.Cu) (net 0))
 (segment (start 144.26 135.08) (end 144.34 135) (width 0.25) (layer B.Cu) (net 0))
 (segment (start 141.12 135.08) (end 144.26 135.08) (width 2.2) (layer B.Cu) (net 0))
 (segment (start 144.34 139.84) (end 144.34 135) (width 2.2) (layer B.Cu) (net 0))
 (segment (start 150.5 144.9525) (end 150.5 145) (width 0.25) (layer B.Cu) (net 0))
 (segment (start 154.5 140.9525) (end 150.5 144.9525) (width 2) (layer B.Cu) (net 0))
 (segment (start 154.5 135) (end 154.5 140.9525) (width 2.2) (layer B.Cu) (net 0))
 (segment (start 144.34 139.84) (end 144.34 143.84) (width 2.2) (layer B.Cu) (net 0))
 (segment (start 145.42 144.92) (end 145.42 145) (width 0.25) (layer B.Cu) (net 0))
 (segment (start 144.34 143.84) (end 145.42 144.92) (width 2.2) (layer B.Cu) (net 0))
 (segment (start 154.5 141) (end 150.5 145) (width 2) (layer F.Cu) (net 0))
 (segment (start 154.5 135) (end 154.5 141) (width 2.2) (layer F.Cu) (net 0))
 (segment (start 154.5 130) (end 153.36863 130) (width 2.2) (layer F.Cu) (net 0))
 (segment (start 149.5 132.5) (end 149.5 140) (width 2.2) (layer B.Cu) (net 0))
 (segment (start 152 130) (end 149.5 132.5) (width 2.2) (layer F.Cu) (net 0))
 (segment (start 149.5 140) (end 147.96 141.54) (width 2.2) (layer B.Cu) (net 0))
 (segment (start 154.5 130) (end 152 130) (width 2.2) (layer B.Cu) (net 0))
 (segment (start 153.36863 130) (end 152 130) (width 2.2) (layer F.Cu) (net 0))
 (segment (start 147.96 141.54) (end 147.96 145) (width 2.2) (layer B.Cu) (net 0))
 (segment (start 152 130) (end 149.5 132.5) (width 2.2) (layer B.Cu) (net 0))
 (segment (start 149.5 132.5) (end 149.5 139.5) (width 2.2) (layer F.Cu) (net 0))
 (segment (start 149.5 139.5) (end 149.5 140) (width 2.2) (layer F.Cu) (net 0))
 (segment (start 149.5 140) (end 148 141.5) (width 2.2) (layer F.Cu) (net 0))
 (segment (start 148 141.5) (end 148 143.5) (width 2.2) (layer F.Cu) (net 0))
 (segment (start 147.96 143.54) (end 147.96 143.96) (width 2.2) (layer F.Cu) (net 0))
 (segment (start 148 143.5) (end 147.96 143.54) (width 0.25) (layer F.Cu) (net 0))
 (segment (start 144.34 143.92) (end 145.42 145) (width 2.2) (layer F.Cu) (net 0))
 (segment (start 144.34 135) (end 144.34 143.92) (width 2.2) (layer F.Cu) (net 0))
 (segment (start 142 130) (end 144.34 130) (width 2.2) (layer B.Cu) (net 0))
 (segment (start 141.12 130) (end 142 130) (width 1.6) (layer B.Cu) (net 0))
 (segment (start 144.26 135.08) (end 144.34 135) (width 0.25) (layer F.Cu) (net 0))
 (segment (start 141.12 135.08) (end 144.26 135.08) (width 2.2) (layer F.Cu) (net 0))
 (segment (start 144.34 130) (end 143 130) (width 0.25) (layer F.Cu) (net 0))
 (segment (start 141.12 130) (end 143 130) (width 2.2) (layer F.Cu) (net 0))
 (segment (start 143 130) (end 143.5 130) (width 2.2) (layer F.Cu) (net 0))
 (segment (start 134.95 127.5) (end 133.5 128.95) (width 1) (layer F.Cu) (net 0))
 (segment (start 133.5 128.95) (end 133.5 130) (width 1) (layer F.Cu) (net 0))
 (segment (start 142.34 127.5) (end 134.95 127.5) (width 1) (layer F.Cu) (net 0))
 (segment (start 144.34 125.5) (end 142.34 127.5) (width 1) (layer F.Cu) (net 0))
 (segment (start 180.16 125.5) (end 180.5 125.84) (width 0.25) (layer B.Cu) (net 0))
 (segment (start 154.5 125.5) (end 180.16 125.5) (width 2.2) (layer B.Cu) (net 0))
 (segment (start 179.58 130) (end 180.5 130.92) (width 2.2) (layer B.Cu) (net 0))
 (segment (start 154.5 130) (end 179.58 130) (width 2.2) (layer B.Cu) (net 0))
 (segment (start 180.5 136) (end 180.5 141.92) (width 2.2) (layer B.Cu) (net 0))
 (segment (start 175 147) (end 180.5 147) (width 2.2) (layer B.Cu) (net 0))
 (segment (start 174 146) (end 175 147) (width 2.2) (layer B.Cu) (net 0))
 (segment (start 174 137) (end 174 146) (width 2.2) (layer B.Cu) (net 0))
 (segment (start 154.5 135) (end 172 135) (width 2.2) (layer B.Cu) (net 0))
 (segment (start 172 135) (end 174 137) (width 2.2) (layer B.Cu) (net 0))
 (segment (start 180.5 147) (end 178.75 147) (width 2) (layer F.Cu) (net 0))
 (segment (start 178.75 147) (end 175 147) (width 2) (layer F.Cu) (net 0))
 (segment (start 175 147) (end 174 146) (width 2) (layer F.Cu) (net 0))
 (segment (start 174 137) (end 172 135) (width 2) (layer F.Cu) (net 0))
 (segment (start 172 135) (end 154.5 135) (width 2) (layer F.Cu) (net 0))
 (segment (start 174 137) (end 174 139) (width 2) (layer F.Cu) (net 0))
 (segment (start 174 146) (end 174 139) (width 2) (layer F.Cu) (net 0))
 (segment (start 174 139) (end 174 138) (width 0.25) (layer F.Cu) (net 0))
 (segment (start 154.5 130) (end 179 130) (width 2) (layer F.Cu) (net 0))
 (segment (start 180.16 125.5) (end 180.5 125.84) (width 0.25) (layer F.Cu) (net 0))
 (segment (start 154.5 125.5) (end 180.16 125.5) (width 2) (layer F.Cu) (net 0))
 (segment (start 180.5 136) (end 180.5 137.75) (width 2) (layer F.Cu) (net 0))
 (segment (start 180.5 137.75) (end 180.5 140.5) (width 2) (layer F.Cu) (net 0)))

